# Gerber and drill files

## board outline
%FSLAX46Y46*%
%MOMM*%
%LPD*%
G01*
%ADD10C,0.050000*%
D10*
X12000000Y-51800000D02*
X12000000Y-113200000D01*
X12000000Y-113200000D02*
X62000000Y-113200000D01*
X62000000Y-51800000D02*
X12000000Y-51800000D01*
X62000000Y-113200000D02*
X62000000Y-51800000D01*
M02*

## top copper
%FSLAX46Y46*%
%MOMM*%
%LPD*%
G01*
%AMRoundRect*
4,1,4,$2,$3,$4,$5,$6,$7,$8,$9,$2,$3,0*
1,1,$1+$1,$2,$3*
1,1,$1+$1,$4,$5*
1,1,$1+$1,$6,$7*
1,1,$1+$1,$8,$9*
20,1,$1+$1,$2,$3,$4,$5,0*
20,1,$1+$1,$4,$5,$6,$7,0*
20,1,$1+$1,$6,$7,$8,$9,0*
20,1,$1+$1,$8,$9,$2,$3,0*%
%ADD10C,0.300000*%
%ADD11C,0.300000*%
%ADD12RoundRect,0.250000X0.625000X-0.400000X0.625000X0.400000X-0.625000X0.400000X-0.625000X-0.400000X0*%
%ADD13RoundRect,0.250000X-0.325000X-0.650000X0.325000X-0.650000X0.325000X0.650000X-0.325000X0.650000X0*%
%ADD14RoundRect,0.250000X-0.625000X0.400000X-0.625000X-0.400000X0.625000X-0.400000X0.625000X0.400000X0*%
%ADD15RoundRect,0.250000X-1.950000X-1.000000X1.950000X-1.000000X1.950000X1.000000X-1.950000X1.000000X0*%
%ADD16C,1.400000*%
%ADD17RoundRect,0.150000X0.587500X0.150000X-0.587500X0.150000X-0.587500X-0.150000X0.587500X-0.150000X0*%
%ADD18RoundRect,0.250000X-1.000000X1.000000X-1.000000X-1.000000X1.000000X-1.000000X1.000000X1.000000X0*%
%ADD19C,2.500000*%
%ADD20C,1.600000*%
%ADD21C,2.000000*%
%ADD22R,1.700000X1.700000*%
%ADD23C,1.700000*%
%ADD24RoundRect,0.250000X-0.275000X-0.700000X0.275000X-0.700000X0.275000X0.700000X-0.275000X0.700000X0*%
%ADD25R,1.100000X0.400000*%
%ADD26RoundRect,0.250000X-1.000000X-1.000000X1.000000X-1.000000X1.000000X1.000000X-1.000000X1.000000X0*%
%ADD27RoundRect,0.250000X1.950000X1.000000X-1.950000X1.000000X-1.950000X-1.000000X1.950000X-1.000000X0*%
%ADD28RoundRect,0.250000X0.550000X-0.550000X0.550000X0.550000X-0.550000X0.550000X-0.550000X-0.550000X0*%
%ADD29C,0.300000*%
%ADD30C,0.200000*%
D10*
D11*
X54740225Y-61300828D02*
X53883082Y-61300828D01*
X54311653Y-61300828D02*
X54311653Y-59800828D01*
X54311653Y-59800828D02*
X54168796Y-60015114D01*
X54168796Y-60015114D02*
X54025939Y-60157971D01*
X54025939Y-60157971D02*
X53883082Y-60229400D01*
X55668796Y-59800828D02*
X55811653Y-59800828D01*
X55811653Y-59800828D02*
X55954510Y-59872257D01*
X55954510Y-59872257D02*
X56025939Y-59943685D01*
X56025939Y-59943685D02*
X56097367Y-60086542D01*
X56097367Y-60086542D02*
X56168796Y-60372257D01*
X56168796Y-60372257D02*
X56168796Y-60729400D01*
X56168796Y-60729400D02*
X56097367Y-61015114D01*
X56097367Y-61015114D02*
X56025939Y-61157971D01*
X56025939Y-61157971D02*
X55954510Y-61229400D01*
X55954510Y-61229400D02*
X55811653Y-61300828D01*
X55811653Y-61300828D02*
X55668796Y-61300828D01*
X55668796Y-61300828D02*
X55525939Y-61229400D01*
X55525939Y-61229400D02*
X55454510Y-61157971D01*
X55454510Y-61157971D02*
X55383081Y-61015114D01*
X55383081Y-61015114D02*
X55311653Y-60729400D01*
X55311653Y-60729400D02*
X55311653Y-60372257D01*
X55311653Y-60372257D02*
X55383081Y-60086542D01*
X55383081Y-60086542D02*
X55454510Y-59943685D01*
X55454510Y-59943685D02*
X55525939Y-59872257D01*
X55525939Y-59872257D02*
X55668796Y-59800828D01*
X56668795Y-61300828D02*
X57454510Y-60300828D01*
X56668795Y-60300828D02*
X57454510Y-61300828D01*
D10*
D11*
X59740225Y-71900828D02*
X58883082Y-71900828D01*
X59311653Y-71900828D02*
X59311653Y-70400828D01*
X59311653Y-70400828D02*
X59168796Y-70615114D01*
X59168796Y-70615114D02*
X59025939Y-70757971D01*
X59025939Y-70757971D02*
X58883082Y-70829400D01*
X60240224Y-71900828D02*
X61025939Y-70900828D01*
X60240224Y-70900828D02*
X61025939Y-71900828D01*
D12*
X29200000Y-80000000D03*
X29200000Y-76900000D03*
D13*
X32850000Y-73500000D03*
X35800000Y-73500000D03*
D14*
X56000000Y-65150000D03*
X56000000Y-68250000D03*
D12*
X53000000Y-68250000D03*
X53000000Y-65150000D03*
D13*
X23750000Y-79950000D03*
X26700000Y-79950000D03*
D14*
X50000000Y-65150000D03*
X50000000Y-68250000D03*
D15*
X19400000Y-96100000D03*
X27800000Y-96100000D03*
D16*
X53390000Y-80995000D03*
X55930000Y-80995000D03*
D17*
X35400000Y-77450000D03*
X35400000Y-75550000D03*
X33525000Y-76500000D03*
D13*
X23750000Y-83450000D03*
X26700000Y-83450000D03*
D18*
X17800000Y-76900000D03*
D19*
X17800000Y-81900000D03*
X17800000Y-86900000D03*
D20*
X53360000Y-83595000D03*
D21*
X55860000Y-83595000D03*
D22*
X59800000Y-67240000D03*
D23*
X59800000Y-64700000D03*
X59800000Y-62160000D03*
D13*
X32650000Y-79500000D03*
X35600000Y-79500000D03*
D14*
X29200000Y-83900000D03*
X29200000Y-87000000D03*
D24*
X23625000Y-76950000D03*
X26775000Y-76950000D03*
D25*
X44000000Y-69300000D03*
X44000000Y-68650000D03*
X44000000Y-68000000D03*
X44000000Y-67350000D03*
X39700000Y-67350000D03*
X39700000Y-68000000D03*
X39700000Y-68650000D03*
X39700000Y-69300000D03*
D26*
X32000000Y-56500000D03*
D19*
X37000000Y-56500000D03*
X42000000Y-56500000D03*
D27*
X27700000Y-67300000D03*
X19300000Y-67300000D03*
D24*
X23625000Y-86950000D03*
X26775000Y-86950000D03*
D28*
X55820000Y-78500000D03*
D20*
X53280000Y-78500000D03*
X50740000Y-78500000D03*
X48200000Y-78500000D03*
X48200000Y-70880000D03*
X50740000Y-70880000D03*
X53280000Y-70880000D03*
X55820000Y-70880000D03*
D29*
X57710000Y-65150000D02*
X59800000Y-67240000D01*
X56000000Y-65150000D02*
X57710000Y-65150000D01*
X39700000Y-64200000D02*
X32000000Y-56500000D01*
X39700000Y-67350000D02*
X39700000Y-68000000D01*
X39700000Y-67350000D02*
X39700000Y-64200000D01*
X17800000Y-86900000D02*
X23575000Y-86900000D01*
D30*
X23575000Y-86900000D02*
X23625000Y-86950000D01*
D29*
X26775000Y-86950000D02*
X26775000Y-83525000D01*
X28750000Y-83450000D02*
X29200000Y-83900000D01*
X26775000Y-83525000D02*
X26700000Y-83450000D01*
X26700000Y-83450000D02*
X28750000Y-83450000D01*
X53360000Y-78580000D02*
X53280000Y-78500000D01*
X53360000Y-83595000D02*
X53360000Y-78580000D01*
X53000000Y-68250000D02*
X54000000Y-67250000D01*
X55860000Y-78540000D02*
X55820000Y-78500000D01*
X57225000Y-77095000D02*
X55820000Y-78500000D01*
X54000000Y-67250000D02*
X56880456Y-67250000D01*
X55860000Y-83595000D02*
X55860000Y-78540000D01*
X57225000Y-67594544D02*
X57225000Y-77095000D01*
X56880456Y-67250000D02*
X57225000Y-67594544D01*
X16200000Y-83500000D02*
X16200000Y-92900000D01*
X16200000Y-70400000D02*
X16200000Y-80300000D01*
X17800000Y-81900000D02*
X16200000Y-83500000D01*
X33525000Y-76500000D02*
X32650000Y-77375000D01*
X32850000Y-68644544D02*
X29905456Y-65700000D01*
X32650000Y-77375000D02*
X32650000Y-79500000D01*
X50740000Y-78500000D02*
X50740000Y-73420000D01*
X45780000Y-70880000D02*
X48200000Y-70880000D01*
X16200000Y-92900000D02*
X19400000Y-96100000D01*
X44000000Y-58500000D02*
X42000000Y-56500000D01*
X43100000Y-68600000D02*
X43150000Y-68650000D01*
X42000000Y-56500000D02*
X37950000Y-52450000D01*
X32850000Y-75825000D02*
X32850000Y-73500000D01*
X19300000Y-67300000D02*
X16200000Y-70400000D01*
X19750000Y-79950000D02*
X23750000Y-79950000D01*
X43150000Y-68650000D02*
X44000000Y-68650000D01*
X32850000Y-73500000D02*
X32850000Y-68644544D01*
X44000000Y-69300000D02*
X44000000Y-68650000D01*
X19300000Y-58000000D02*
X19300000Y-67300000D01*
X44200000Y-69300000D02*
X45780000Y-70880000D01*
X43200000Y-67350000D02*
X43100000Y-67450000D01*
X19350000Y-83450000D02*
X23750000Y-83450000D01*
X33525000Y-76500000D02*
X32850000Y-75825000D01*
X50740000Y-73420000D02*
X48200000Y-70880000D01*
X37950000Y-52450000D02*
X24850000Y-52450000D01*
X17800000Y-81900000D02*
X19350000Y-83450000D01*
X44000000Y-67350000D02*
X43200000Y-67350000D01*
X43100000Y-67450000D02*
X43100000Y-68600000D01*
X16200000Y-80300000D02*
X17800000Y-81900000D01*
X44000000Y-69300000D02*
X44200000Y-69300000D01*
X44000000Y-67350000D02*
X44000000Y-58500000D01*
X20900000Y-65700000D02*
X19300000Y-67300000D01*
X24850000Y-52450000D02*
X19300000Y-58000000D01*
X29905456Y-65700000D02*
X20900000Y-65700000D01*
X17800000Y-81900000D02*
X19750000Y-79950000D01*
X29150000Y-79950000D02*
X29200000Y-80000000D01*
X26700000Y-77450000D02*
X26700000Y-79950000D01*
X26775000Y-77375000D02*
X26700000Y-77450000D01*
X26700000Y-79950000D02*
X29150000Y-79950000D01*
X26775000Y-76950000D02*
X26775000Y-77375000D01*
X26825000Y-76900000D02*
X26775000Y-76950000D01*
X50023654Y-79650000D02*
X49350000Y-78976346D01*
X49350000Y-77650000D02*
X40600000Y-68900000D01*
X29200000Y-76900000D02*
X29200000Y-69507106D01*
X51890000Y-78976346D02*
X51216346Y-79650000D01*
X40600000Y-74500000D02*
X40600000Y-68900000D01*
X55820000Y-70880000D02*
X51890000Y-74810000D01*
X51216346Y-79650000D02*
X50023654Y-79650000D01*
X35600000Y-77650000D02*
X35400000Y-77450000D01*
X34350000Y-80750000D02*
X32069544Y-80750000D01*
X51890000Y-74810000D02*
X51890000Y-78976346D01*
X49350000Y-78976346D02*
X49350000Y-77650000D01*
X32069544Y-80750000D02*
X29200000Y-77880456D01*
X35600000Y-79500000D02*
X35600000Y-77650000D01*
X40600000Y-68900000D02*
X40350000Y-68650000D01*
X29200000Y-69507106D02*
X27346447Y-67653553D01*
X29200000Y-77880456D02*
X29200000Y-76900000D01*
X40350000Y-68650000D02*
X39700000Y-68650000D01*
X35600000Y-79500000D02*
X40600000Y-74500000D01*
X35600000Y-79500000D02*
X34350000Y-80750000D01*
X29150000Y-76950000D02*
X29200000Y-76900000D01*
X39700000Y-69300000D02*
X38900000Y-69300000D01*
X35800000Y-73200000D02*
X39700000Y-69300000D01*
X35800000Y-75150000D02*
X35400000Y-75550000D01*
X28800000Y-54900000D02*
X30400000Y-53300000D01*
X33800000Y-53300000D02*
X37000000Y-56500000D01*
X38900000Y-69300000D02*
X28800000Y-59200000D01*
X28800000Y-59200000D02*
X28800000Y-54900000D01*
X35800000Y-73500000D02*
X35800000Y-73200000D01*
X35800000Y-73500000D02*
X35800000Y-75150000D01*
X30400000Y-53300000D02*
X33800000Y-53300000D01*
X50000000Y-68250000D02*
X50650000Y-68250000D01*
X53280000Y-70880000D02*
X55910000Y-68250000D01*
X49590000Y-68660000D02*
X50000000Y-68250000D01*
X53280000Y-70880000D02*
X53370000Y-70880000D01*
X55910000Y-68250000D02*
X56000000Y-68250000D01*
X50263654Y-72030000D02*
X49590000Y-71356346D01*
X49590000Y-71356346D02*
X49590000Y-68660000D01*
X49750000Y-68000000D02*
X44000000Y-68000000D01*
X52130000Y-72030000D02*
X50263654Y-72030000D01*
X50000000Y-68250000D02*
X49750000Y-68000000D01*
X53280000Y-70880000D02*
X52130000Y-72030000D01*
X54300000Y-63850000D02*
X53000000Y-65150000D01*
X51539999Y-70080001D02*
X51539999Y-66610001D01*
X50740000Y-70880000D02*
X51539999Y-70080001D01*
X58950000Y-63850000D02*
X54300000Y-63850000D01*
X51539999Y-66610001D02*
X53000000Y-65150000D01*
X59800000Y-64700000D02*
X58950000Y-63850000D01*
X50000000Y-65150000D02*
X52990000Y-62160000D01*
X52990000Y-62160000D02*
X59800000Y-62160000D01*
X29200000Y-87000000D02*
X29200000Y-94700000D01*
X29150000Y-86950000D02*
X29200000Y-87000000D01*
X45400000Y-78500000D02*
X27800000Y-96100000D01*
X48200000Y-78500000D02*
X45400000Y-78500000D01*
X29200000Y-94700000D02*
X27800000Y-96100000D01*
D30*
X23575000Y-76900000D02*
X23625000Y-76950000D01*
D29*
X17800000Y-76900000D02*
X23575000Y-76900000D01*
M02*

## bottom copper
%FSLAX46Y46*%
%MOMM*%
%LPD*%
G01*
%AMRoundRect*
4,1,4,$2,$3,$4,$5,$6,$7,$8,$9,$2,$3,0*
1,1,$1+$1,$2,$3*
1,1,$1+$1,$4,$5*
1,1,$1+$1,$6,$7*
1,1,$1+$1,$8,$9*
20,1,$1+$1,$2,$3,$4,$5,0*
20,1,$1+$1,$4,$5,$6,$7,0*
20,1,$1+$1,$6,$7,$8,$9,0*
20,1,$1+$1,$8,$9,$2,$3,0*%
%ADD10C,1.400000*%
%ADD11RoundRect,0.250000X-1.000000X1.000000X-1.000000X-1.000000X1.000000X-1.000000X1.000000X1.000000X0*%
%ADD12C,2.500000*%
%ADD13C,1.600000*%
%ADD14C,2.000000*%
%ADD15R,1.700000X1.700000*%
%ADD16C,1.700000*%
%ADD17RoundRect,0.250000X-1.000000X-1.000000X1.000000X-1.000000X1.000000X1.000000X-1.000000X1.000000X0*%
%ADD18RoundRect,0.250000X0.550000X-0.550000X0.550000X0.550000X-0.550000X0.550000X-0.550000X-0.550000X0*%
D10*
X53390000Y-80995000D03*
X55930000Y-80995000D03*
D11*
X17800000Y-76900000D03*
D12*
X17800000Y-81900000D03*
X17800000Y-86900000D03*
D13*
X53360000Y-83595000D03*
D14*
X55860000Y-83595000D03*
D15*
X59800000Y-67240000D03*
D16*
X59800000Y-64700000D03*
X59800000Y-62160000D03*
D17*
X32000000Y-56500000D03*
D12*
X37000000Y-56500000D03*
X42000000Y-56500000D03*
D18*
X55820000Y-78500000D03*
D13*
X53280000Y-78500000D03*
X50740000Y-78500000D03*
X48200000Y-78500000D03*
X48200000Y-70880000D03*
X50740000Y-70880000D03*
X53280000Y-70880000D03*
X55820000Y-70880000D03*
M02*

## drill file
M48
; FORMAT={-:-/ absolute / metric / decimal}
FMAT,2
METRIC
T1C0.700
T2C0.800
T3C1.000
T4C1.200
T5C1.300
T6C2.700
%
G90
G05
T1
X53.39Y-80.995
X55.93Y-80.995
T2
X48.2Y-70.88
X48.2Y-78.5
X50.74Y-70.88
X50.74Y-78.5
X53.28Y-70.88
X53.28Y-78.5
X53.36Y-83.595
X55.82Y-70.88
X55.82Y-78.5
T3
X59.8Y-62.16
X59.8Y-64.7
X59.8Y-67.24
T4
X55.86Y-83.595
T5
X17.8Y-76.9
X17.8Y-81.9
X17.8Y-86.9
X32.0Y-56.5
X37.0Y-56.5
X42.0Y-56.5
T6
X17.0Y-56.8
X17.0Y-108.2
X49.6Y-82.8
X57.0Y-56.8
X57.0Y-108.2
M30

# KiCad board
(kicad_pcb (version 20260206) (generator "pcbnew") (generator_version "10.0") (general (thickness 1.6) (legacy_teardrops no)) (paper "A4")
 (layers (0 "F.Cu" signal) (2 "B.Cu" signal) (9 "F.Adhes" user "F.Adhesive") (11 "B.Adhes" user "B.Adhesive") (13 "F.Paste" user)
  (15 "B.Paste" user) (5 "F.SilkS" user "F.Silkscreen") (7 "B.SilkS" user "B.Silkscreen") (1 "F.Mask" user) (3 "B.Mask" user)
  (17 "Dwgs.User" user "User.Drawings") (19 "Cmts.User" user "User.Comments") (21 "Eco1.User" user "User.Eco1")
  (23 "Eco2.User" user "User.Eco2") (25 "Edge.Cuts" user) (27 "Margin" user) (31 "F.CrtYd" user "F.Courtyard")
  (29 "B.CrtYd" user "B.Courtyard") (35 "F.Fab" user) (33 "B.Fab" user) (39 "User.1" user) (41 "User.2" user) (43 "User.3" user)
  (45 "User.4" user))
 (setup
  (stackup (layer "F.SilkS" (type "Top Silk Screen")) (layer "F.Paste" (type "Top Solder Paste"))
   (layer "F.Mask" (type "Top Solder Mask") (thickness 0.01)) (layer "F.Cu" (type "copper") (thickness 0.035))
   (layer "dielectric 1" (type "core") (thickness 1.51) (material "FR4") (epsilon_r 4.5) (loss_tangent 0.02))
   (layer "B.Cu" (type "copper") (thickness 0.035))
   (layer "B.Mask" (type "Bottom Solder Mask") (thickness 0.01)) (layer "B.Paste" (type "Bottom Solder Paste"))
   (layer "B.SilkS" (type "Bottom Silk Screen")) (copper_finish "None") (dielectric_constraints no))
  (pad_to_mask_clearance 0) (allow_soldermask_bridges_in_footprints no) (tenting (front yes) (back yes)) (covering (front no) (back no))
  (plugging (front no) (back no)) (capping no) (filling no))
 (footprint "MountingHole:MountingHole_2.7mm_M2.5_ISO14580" (layer "F.Cu") (at 57 56.8 -90)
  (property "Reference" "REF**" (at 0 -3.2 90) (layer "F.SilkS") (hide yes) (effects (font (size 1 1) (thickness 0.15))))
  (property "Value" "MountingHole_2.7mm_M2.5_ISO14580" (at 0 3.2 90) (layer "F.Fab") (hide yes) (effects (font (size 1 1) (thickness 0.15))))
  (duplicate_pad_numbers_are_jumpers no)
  (pad "" np_thru_hole circle (at 0 0 270) (size 2.7 2.7) (drill 2.7) (layers "*.Cu" "*.Mask")))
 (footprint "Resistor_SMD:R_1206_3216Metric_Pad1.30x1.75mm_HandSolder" (layer "F.Cu") (at 29.2 78.45 90)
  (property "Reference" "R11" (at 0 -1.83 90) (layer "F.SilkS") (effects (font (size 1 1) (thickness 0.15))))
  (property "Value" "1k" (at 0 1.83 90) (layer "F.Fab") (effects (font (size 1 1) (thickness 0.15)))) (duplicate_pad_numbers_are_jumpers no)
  (pad "1" smd roundrect (at -1.55 0 90) (size 1.3 1.75) (layers "F.Cu" "F.Mask" "F.Paste") (roundrect_rratio 0.192308)
   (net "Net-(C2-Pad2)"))
  (pad "2" smd roundrect (at 1.55 0 90) (size 1.3 1.75) (layers "F.Cu" "F.Mask" "F.Paste") (roundrect_rratio 0.192308) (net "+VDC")))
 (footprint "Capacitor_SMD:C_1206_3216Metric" (layer "F.Cu") (at 34.325 73.5)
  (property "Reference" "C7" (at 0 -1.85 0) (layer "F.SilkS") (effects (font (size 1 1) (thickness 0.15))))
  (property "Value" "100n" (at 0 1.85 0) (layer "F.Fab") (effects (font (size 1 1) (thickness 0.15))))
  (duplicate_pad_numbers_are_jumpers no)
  (pad "1" smd roundrect (at -1.475 0) (size 1.15 1.8) (layers "F.Cu" "F.Mask" "F.Paste") (roundrect_rratio 0.217391) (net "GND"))
  (pad "2" smd roundrect (at 1.475 0) (size 1.15 1.8) (layers "F.Cu" "F.Mask" "F.Paste") (roundrect_rratio 0.217391) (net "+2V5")))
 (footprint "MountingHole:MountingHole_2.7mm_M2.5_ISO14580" (layer "F.Cu") (at 49.6 82.8 180)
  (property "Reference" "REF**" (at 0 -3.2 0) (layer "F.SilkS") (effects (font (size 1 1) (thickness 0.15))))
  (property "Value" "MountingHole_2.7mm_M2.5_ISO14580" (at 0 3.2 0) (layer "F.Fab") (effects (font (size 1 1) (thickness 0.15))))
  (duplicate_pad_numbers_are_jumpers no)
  (pad "" np_thru_hole circle (at 0 0 180) (size 2.7 2.7) (drill 2.7) (layers "*.Cu" "*.Mask")))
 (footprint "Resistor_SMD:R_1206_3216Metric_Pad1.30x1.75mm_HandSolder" (layer "F.Cu") (at 56 66.7 -90)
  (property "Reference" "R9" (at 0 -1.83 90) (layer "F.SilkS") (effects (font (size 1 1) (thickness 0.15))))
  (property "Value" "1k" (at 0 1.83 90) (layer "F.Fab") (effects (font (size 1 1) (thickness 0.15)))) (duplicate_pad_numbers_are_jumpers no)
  (pad "1" smd roundrect (at -1.55 0 270) (size 1.3 1.75) (layers "F.Cu" "F.Mask" "F.Paste") (roundrect_rratio 0.192308)
   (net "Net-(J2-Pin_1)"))
  (pad "2" smd roundrect (at 1.55 0 270) (size 1.3 1.75) (layers "F.Cu" "F.Mask" "F.Paste") (roundrect_rratio 0.192308)
   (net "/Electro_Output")))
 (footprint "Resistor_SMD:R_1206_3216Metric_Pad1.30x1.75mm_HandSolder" (layer "F.Cu") (at 53 66.7 90)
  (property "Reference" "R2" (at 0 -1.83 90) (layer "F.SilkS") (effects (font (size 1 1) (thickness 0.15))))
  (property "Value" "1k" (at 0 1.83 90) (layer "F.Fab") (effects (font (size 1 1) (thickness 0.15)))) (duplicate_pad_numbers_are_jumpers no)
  (pad "1" smd roundrect (at -1.55 0 90) (size 1.3 1.75) (layers "F.Cu" "F.Mask" "F.Paste") (roundrect_rratio 0.192308)
   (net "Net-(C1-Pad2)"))
  (pad "2" smd roundrect (at 1.55 0 90) (size 1.3 1.75) (layers "F.Cu" "F.Mask" "F.Paste") (roundrect_rratio 0.192308)
   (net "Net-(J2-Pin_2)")))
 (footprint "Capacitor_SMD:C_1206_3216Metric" (layer "F.Cu") (at 25.225 79.95)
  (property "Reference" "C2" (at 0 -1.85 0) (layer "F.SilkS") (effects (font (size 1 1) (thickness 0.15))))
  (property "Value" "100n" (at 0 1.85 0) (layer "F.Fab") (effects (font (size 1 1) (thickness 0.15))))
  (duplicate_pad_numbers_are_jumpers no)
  (pad "1" smd roundrect (at -1.475 0) (size 1.15 1.8) (layers "F.Cu" "F.Mask" "F.Paste") (roundrect_rratio 0.217391) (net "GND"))
  (pad "2" smd roundrect (at 1.475 0) (size 1.15 1.8) (layers "F.Cu" "F.Mask" "F.Paste") (roundrect_rratio 0.217391) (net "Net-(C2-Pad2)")))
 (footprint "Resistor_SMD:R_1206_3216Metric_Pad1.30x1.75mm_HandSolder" (layer "F.Cu") (at 50 66.7 -90)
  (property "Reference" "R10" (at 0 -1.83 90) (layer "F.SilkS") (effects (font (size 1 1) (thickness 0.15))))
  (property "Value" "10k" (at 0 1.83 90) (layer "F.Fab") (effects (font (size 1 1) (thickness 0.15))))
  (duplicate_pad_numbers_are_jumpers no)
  (pad "1" smd roundrect (at -1.55 0 270) (size 1.3 1.75) (layers "F.Cu" "F.Mask" "F.Paste") (roundrect_rratio 0.192308)
   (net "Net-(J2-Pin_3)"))
  (pad "2" smd roundrect (at 1.55 0 270) (size 1.3 1.75) (layers "F.Cu" "F.Mask" "F.Paste") (roundrect_rratio 0.192308)
   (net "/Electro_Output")))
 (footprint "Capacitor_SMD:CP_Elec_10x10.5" (layer "F.Cu") (at 23.6 96.1)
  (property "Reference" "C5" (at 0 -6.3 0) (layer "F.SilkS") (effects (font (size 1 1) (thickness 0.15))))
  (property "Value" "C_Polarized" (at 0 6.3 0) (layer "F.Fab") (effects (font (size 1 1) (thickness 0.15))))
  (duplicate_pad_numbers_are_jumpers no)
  (pad "1" smd roundrect (at -4.2 0) (size 4.4 2.5) (layers "F.Cu" "F.Mask" "F.Paste") (roundrect_rratio 0.1) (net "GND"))
  (pad "2" smd roundrect (at 4.2 0) (size 4.4 2.5) (layers "F.Cu" "F.Mask" "F.Paste") (roundrect_rratio 0.1) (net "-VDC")))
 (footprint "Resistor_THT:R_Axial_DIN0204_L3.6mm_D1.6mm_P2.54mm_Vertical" (layer "F.Cu") (at 53.39 80.995)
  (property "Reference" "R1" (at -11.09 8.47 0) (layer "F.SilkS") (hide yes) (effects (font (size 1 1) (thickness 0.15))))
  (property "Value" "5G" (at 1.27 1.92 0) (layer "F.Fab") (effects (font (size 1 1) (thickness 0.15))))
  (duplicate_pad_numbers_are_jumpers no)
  (pad "1" thru_hole circle (at 0 0) (size 1.4 1.4) (drill 0.7) (layers "*.Cu" "*.Mask") (remove_unused_layers no) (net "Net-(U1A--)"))
  (pad "2" thru_hole circle (at 2.54 0) (size 1.4 1.4) (drill 0.7) (layers "*.Cu" "*.Mask") (remove_unused_layers no) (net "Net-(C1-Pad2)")))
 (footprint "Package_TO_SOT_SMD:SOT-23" (layer "F.Cu") (at 34.4625 76.5 180)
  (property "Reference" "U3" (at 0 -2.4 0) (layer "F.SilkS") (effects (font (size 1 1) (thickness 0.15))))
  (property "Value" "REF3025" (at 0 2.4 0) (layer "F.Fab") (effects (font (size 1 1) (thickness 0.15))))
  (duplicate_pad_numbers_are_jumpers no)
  (pad "1" smd roundrect (at -0.9375 -0.95 180) (size 1.475 0.6) (layers "F.Cu" "F.Mask" "F.Paste") (roundrect_rratio 0.25) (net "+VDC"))
  (pad "2" smd roundrect (at -0.9375 0.95 180) (size 1.475 0.6) (layers "F.Cu" "F.Mask" "F.Paste") (roundrect_rratio 0.25) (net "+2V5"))
  (pad "3" smd roundrect (at 0.9375 0 180) (size 1.475 0.6) (layers "F.Cu" "F.Mask" "F.Paste") (roundrect_rratio 0.25) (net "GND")))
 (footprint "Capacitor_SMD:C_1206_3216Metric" (layer "F.Cu") (at 25.225 83.45)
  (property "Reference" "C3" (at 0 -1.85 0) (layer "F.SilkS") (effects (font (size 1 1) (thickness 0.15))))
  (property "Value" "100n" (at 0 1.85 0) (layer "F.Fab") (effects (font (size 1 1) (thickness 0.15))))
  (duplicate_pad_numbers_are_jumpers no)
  (pad "1" smd roundrect (at -1.475 0) (size 1.15 1.8) (layers "F.Cu" "F.Mask" "F.Paste") (roundrect_rratio 0.217391) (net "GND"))
  (pad "2" smd roundrect (at 1.475 0) (size 1.15 1.8) (layers "F.Cu" "F.Mask" "F.Paste") (roundrect_rratio 0.217391) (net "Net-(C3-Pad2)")))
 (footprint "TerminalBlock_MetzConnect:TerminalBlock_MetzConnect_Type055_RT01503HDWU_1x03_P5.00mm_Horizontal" (layer "F.Cu")
  (at 17.8 76.9 -90)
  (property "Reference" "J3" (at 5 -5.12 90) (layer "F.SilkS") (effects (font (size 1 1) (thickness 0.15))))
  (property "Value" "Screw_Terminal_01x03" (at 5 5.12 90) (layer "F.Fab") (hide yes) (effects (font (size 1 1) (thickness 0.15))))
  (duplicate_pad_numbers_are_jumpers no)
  (pad "1" thru_hole roundrect (at 0 0 270) (size 2.5 2.5) (drill 1.3) (layers "*.Cu" "*.Mask") (remove_unused_layers no)
   (roundrect_rratio 0.1) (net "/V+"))
  (pad "2" thru_hole circle (at 5 0 270) (size 2.5 2.5) (drill 1.3) (layers "*.Cu" "*.Mask") (remove_unused_layers no) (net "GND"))
  (pad "3" thru_hole circle (at 10 0 270) (size 2.5 2.5) (drill 1.3) (layers "*.Cu" "*.Mask") (remove_unused_layers no) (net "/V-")))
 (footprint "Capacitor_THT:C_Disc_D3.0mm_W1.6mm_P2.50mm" (layer "F.Cu") (at 53.36 83.595)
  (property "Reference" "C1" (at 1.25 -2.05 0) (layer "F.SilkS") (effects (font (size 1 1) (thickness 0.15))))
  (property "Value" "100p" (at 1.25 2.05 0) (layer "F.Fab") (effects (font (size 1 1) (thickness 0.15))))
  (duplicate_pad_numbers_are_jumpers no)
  (pad "1" thru_hole circle (at 0 0) (size 1.6 1.6) (drill 0.8) (layers "*.Cu" "*.Mask") (remove_unused_layers no) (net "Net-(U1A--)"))
  (pad "2" thru_hole circle (at 2.5 0) (size 2 2) (drill 1.2) (layers "*.Cu" "*.Mask") (remove_unused_layers no) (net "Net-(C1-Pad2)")))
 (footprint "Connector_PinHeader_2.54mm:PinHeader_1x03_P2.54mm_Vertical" (layer "F.Cu") (at 59.8 67.24 180)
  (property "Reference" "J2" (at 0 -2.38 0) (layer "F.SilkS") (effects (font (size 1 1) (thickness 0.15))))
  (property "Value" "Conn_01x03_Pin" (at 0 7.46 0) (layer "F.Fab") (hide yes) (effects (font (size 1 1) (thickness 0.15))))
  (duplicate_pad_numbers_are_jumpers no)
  (pad "1" thru_hole rect (at 0 0 180) (size 1.7 1.7) (drill 1) (layers "*.Cu" "*.Mask") (remove_unused_layers no) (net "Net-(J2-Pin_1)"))
  (pad "2" thru_hole circle (at 0 2.54 180) (size 1.7 1.7) (drill 1) (layers "*.Cu" "*.Mask") (remove_unused_layers no)
   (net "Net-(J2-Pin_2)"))
  (pad "3" thru_hole circle (at 0 5.08 180) (size 1.7 1.7) (drill 1) (layers "*.Cu" "*.Mask") (remove_unused_layers no)
   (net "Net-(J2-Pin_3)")))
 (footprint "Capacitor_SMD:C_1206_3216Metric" (layer "F.Cu") (at 34.125 79.5)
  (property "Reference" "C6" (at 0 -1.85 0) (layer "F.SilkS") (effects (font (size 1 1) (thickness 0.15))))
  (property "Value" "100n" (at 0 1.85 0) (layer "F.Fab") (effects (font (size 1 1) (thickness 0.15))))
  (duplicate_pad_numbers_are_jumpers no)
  (pad "1" smd roundrect (at -1.475 0) (size 1.15 1.8) (layers "F.Cu" "F.Mask" "F.Paste") (roundrect_rratio 0.217391) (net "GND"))
  (pad "2" smd roundrect (at 1.475 0) (size 1.15 1.8) (layers "F.Cu" "F.Mask" "F.Paste") (roundrect_rratio 0.217391) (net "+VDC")))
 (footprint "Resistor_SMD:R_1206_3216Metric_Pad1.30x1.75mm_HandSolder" (layer "F.Cu") (at 29.2 85.45 -90)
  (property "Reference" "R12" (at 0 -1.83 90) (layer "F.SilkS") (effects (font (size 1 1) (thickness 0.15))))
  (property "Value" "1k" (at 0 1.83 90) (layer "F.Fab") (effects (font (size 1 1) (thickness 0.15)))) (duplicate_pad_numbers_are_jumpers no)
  (pad "1" smd roundrect (at -1.55 0 270) (size 1.3 1.75) (layers "F.Cu" "F.Mask" "F.Paste") (roundrect_rratio 0.192308)
   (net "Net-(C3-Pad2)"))
  (pad "2" smd roundrect (at 1.55 0 270) (size 1.3 1.75) (layers "F.Cu" "F.Mask" "F.Paste") (roundrect_rratio 0.192308) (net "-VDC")))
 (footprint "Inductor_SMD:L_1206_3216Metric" (layer "F.Cu") (at 25.2 76.95)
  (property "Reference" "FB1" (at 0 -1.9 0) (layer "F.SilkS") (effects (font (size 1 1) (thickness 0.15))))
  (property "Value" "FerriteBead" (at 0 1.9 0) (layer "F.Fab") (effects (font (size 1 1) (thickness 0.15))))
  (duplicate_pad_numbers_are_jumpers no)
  (pad "1" smd roundrect (at -1.575 0) (size 1.05 1.9) (layers "F.Cu" "F.Mask" "F.Paste") (roundrect_rratio 0.238095) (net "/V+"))
  (pad "2" smd roundrect (at 1.575 0) (size 1.05 1.9) (layers "F.Cu" "F.Mask" "F.Paste") (roundrect_rratio 0.238095) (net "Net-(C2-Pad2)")))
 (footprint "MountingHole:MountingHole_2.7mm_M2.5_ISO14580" (layer "F.Cu") (at 57 108.2 -90)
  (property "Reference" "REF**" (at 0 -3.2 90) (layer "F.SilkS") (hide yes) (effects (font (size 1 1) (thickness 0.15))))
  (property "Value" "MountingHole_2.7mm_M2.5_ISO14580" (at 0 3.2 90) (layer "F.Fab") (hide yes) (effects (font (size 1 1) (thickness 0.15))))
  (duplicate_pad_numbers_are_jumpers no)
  (pad "" np_thru_hole circle (at 0 0 270) (size 2.7 2.7) (drill 2.7) (layers "*.Cu" "*.Mask")))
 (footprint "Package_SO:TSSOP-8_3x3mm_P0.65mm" (layer "F.Cu") (at 41.85 68.325 180)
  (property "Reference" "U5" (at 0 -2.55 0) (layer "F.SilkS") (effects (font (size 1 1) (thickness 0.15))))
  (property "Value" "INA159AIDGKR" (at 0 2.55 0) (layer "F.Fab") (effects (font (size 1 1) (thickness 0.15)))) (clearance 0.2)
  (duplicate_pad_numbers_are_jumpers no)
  (pad "1" smd rect (at -2.15 -0.975 180) (size 1.1 0.4) (layers "F.Cu" "F.Mask" "F.Paste") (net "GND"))
  (pad "2" smd rect (at -2.15 -0.325 180) (size 1.1 0.4) (layers "F.Cu" "F.Mask" "F.Paste") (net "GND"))
  (pad "3" smd rect (at -2.15 0.325 180) (size 1.1 0.4) (layers "F.Cu" "F.Mask" "F.Paste") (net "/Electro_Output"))
  (pad "4" smd rect (at -2.15 0.975 180) (size 1.1 0.4) (layers "F.Cu" "F.Mask" "F.Paste") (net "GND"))
  (pad "5" smd rect (at 2.15 0.975 180) (size 1.1 0.4) (layers "F.Cu" "F.Mask" "F.Paste") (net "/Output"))
  (pad "6" smd rect (at 2.15 0.325 180) (size 1.1 0.4) (layers "F.Cu" "F.Mask" "F.Paste") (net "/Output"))
  (pad "7" smd rect (at 2.15 -0.325 180) (size 1.1 0.4) (layers "F.Cu" "F.Mask" "F.Paste") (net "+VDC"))
  (pad "8" smd rect (at 2.15 -0.975 180) (size 1.1 0.4) (layers "F.Cu" "F.Mask" "F.Paste") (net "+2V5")))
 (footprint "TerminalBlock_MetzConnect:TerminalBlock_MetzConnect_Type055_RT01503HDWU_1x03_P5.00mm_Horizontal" (layer "F.Cu") (at 32 56.5)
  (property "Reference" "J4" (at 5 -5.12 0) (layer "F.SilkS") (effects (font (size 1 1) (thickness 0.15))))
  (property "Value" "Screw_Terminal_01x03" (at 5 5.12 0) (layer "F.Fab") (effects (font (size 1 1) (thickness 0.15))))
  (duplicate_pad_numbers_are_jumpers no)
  (pad "1" thru_hole roundrect (at 0 0) (size 2.5 2.5) (drill 1.3) (layers "*.Cu" "*.Mask") (remove_unused_layers no) (roundrect_rratio 0.1)
   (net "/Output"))
  (pad "2" thru_hole circle (at 5 0) (size 2.5 2.5) (drill 1.3) (layers "*.Cu" "*.Mask") (remove_unused_layers no) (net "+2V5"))
  (pad "3" thru_hole circle (at 10 0) (size 2.5 2.5) (drill 1.3) (layers "*.Cu" "*.Mask") (remove_unused_layers no) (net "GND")))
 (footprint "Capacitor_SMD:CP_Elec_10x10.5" (layer "F.Cu") (at 23.5 67.3 180)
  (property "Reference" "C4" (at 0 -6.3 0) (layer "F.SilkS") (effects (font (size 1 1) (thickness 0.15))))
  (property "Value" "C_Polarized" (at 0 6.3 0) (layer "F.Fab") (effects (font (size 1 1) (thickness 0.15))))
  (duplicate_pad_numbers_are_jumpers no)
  (pad "1" smd roundrect (at -4.2 0 180) (size 4.4 2.5) (layers "F.Cu" "F.Mask" "F.Paste") (roundrect_rratio 0.1) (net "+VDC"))
  (pad "2" smd roundrect (at 4.2 0 180) (size 4.4 2.5) (layers "F.Cu" "F.Mask" "F.Paste") (roundrect_rratio 0.1) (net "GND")))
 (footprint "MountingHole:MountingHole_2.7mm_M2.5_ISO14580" (layer "F.Cu") (at 17 108.2 -90)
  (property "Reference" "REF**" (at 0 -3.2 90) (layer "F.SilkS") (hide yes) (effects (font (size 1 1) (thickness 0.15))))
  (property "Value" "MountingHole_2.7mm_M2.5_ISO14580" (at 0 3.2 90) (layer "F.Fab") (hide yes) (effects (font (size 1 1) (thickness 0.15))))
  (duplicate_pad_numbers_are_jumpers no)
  (pad "" np_thru_hole circle (at 0 0 270) (size 2.7 2.7) (drill 2.7) (layers "*.Cu" "*.Mask")))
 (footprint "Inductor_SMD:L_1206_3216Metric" (layer "F.Cu") (at 25.2 86.95)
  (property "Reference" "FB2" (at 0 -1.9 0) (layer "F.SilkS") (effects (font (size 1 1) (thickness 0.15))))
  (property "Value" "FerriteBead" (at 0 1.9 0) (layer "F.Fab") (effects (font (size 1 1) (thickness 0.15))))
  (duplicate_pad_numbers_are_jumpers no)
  (pad "1" smd roundrect (at -1.575 0) (size 1.05 1.9) (layers "F.Cu" "F.Mask" "F.Paste") (roundrect_rratio 0.238095) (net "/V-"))
  (pad "2" smd roundrect (at 1.575 0) (size 1.05 1.9) (layers "F.Cu" "F.Mask" "F.Paste") (roundrect_rratio 0.238095) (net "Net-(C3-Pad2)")))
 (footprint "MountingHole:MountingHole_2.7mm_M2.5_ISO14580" (layer "F.Cu") (at 17 56.8 -90)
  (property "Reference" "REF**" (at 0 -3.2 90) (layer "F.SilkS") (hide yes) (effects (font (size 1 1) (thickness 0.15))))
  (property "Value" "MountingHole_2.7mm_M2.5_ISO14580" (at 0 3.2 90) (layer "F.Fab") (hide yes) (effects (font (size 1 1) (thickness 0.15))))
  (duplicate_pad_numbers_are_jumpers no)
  (pad "" np_thru_hole circle (at 0 0 270) (size 2.7 2.7) (drill 2.7) (layers "*.Cu" "*.Mask")))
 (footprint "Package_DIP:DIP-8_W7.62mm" (layer "B.Cu") (at 55.82 78.5 90)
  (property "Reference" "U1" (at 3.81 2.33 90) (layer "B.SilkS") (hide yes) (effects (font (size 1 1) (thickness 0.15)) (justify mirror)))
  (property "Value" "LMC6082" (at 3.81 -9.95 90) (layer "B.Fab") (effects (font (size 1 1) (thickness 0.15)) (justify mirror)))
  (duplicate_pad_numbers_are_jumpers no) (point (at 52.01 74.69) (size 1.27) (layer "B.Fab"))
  (pad "1" thru_hole roundrect (at 0 0 90) (size 1.6 1.6) (drill 0.8) (layers "*.Cu" "*.Mask") (remove_unused_layers no)
   (roundrect_rratio 0.15625) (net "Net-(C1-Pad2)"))
  (pad "2" thru_hole circle (at 0 -2.54 90) (size 1.6 1.6) (drill 0.8) (layers "*.Cu" "*.Mask") (remove_unused_layers no)
   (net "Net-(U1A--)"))
  (pad "3" thru_hole circle (at 0 -5.08 90) (size 1.6 1.6) (drill 0.8) (layers "*.Cu" "*.Mask") (remove_unused_layers no) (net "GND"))
  (pad "4" thru_hole circle (at 0 -7.62 90) (size 1.6 1.6) (drill 0.8) (layers "*.Cu" "*.Mask") (remove_unused_layers no) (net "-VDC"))
  (pad "5" thru_hole circle (at 7.62 -7.62 90) (size 1.6 1.6) (drill 0.8) (layers "*.Cu" "*.Mask") (remove_unused_layers no) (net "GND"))
  (pad "6" thru_hole circle (at 7.62 -5.08 90) (size 1.6 1.6) (drill 0.8) (layers "*.Cu" "*.Mask") (remove_unused_layers no)
   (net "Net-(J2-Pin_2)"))
  (pad "7" thru_hole circle (at 7.62 -2.54 90) (size 1.6 1.6) (drill 0.8) (layers "*.Cu" "*.Mask") (remove_unused_layers no)
   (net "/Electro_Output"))
  (pad "8" thru_hole circle (at 7.62 0 90) (size 1.6 1.6) (drill 0.8) (layers "*.Cu" "*.Mask") (remove_unused_layers no) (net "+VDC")))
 (gr_line (start 12 51.8) (end 12 113.2) (stroke (width 0.05) (type default)) (layer "Edge.Cuts"))
 (gr_line (start 12 113.2) (end 62 113.2) (stroke (width 0.05) (type default)) (layer "Edge.Cuts"))
 (gr_line (start 62 51.8) (end 12 51.8) (stroke (width 0.05) (type default)) (layer "Edge.Cuts"))
 (gr_line (start 62 113.2) (end 62 51.8) (stroke (width 0.05) (type default)) (layer "Edge.Cuts"))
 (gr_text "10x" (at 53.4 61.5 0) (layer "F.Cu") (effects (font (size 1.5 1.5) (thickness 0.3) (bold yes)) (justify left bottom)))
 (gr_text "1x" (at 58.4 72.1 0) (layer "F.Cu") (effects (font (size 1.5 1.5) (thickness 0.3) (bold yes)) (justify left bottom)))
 (segment (start 57.71 65.15) (end 59.8 67.24) (width 0.3) (layer "F.Cu") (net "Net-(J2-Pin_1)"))
 (segment (start 56 65.15) (end 57.71 65.15) (width 0.3) (layer "F.Cu") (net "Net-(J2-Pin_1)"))
 (segment (start 39.7 64.2) (end 32 56.5) (width 0.3) (layer "F.Cu") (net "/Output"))
 (segment (start 39.7 67.35) (end 39.7 68) (width 0.3) (layer "F.Cu") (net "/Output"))
 (segment (start 39.7 67.35) (end 39.7 64.2) (width 0.3) (layer "F.Cu") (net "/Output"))
 (segment (start 17.8 86.9) (end 23.575 86.9) (width 0.3) (layer "F.Cu") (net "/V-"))
 (segment (start 23.575 86.9) (end 23.625 86.95) (width 0.2) (layer "F.Cu") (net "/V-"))
 (segment (start 26.775 86.95) (end 26.775 83.525) (width 0.3) (layer "F.Cu") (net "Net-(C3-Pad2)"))
 (segment (start 28.75 83.45) (end 29.2 83.9) (width 0.3) (layer "F.Cu") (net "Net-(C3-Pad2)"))
 (segment (start 26.775 83.525) (end 26.7 83.45) (width 0.3) (layer "F.Cu") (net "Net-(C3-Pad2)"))
 (segment (start 26.7 83.45) (end 28.75 83.45) (width 0.3) (layer "F.Cu") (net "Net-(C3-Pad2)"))
 (segment (start 53.36 78.58) (end 53.28 78.5) (width 0.3) (layer "F.Cu") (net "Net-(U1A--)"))
 (segment (start 53.36 83.595) (end 53.36 78.58) (width 0.3) (layer "F.Cu") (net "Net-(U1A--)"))
 (segment (start 53 68.25) (end 54 67.25) (width 0.3) (layer "F.Cu") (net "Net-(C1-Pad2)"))
 (segment (start 55.86 78.54) (end 55.82 78.5) (width 0.3) (layer "F.Cu") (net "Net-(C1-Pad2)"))
 (segment (start 57.225 77.095) (end 55.82 78.5) (width 0.3) (layer "F.Cu") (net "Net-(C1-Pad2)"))
 (segment (start 54 67.25) (end 56.880456 67.25) (width 0.3) (layer "F.Cu") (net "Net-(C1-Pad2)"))
 (segment (start 55.86 83.595) (end 55.86 78.54) (width 0.3) (layer "F.Cu") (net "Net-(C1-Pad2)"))
 (segment (start 57.225 67.594544) (end 57.225 77.095) (width 0.3) (layer "F.Cu") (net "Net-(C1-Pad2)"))
 (segment (start 56.880456 67.25) (end 57.225 67.594544) (width 0.3) (layer "F.Cu") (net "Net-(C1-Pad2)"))
 (segment (start 16.2 83.5) (end 16.2 92.9) (width 0.3) (layer "F.Cu") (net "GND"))
 (segment (start 16.2 70.4) (end 16.2 80.3) (width 0.3) (layer "F.Cu") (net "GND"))
 (segment (start 17.8 81.9) (end 16.2 83.5) (width 0.3) (layer "F.Cu") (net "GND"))
 (segment (start 33.525 76.5) (end 32.65 77.375) (width 0.3) (layer "F.Cu") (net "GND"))
 (segment (start 32.85 68.644544) (end 29.905456 65.7) (width 0.3) (layer "F.Cu") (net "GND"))
 (segment (start 32.65 77.375) (end 32.65 79.5) (width 0.3) (layer "F.Cu") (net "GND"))
 (segment (start 50.74 78.5) (end 50.74 73.42) (width 0.3) (layer "F.Cu") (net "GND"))
 (segment (start 45.78 70.88) (end 48.2 70.88) (width 0.3) (layer "F.Cu") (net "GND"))
 (segment (start 16.2 92.9) (end 19.4 96.1) (width 0.3) (layer "F.Cu") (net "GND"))
 (segment (start 44 58.5) (end 42 56.5) (width 0.3) (layer "F.Cu") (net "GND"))
 (segment (start 43.1 68.6) (end 43.15 68.65) (width 0.3) (layer "F.Cu") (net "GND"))
 (segment (start 42 56.5) (end 37.95 52.45) (width 0.3) (layer "F.Cu") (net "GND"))
 (segment (start 32.85 75.825) (end 32.85 73.5) (width 0.3) (layer "F.Cu") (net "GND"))
 (segment (start 19.3 67.3) (end 16.2 70.4) (width 0.3) (layer "F.Cu") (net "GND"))
 (segment (start 19.75 79.95) (end 23.75 79.95) (width 0.3) (layer "F.Cu") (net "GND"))
 (segment (start 43.15 68.65) (end 44 68.65) (width 0.3) (layer "F.Cu") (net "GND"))
 (segment (start 32.85 73.5) (end 32.85 68.644544) (width 0.3) (layer "F.Cu") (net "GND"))
 (segment (start 44 69.3) (end 44 68.65) (width 0.3) (layer "F.Cu") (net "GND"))
 (segment (start 19.3 58) (end 19.3 67.3) (width 0.3) (layer "F.Cu") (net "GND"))
 (segment (start 44.2 69.3) (end 45.78 70.88) (width 0.3) (layer "F.Cu") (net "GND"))
 (segment (start 43.2 67.35) (end 43.1 67.45) (width 0.3) (layer "F.Cu") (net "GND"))
 (segment (start 19.35 83.45) (end 23.75 83.45) (width 0.3) (layer "F.Cu") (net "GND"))
 (segment (start 33.525 76.5) (end 32.85 75.825) (width 0.3) (layer "F.Cu") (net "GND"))
 (segment (start 50.74 73.42) (end 48.2 70.88) (width 0.3) (layer "F.Cu") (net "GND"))
 (segment (start 37.95 52.45) (end 24.85 52.45) (width 0.3) (layer "F.Cu") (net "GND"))
 (segment (start 17.8 81.9) (end 19.35 83.45) (width 0.3) (layer "F.Cu") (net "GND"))
 (segment (start 44 67.35) (end 43.2 67.35) (width 0.3) (layer "F.Cu") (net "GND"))
 (segment (start 43.1 67.45) (end 43.1 68.6) (width 0.3) (layer "F.Cu") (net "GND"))
 (segment (start 16.2 80.3) (end 17.8 81.9) (width 0.3) (layer "F.Cu") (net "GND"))
 (segment (start 44 69.3) (end 44.2 69.3) (width 0.3) (layer "F.Cu") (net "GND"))
 (segment (start 44 67.35) (end 44 58.5) (width 0.3) (layer "F.Cu") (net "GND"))
 (segment (start 20.9 65.7) (end 19.3 67.3) (width 0.3) (layer "F.Cu") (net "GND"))
 (segment (start 24.85 52.45) (end 19.3 58) (width 0.3) (layer "F.Cu") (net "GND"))
 (segment (start 29.905456 65.7) (end 20.9 65.7) (width 0.3) (layer "F.Cu") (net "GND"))
 (segment (start 17.8 81.9) (end 19.75 79.95) (width 0.3) (layer "F.Cu") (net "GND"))
 (segment (start 29.15 79.95) (end 29.2 80) (width 0.3) (layer "F.Cu") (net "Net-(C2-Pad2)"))
 (segment (start 26.7 77.45) (end 26.7 79.95) (width 0.3) (layer "F.Cu") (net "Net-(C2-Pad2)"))
 (segment (start 26.775 77.375) (end 26.7 77.45) (width 0.3) (layer "F.Cu") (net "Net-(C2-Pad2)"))
 (segment (start 26.7 79.95) (end 29.15 79.95) (width 0.3) (layer "F.Cu") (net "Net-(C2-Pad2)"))
 (segment (start 26.775 76.95) (end 26.775 77.375) (width 0.3) (layer "F.Cu") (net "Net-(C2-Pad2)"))
 (segment (start 26.825 76.9) (end 26.775 76.95) (width 0.3) (layer "F.Cu") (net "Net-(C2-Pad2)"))
 (segment (start 50.023654 79.65) (end 49.35 78.976346) (width 0.3) (layer "F.Cu") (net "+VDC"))
 (segment (start 49.35 77.65) (end 40.6 68.9) (width 0.3) (layer "F.Cu") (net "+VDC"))
 (segment (start 29.2 76.9) (end 29.2 69.507106) (width 0.3) (layer "F.Cu") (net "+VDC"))
 (segment (start 51.89 78.976346) (end 51.216346 79.65) (width 0.3) (layer "F.Cu") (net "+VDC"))
 (segment (start 40.6 74.5) (end 40.6 68.9) (width 0.3) (layer "F.Cu") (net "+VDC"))
 (segment (start 55.82 70.88) (end 51.89 74.81) (width 0.3) (layer "F.Cu") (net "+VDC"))
 (segment (start 51.216346 79.65) (end 50.023654 79.65) (width 0.3) (layer "F.Cu") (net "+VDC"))
 (segment (start 35.6 77.65) (end 35.4 77.45) (width 0.3) (layer "F.Cu") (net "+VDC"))
 (segment (start 34.35 80.75) (end 32.069544 80.75) (width 0.3) (layer "F.Cu") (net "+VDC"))
 (segment (start 51.89 74.81) (end 51.89 78.976346) (width 0.3) (layer "F.Cu") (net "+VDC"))
 (segment (start 49.35 78.976346) (end 49.35 77.65) (width 0.3) (layer "F.Cu") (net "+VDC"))
 (segment (start 32.069544 80.75) (end 29.2 77.880456) (width 0.3) (layer "F.Cu") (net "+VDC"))
 (segment (start 35.6 79.5) (end 35.6 77.65) (width 0.3) (layer "F.Cu") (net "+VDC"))
 (segment (start 40.6 68.9) (end 40.35 68.65) (width 0.3) (layer "F.Cu") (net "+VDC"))
 (segment (start 29.2 69.507106) (end 27.346447 67.653553) (width 0.3) (layer "F.Cu") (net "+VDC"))
 (segment (start 29.2 77.880456) (end 29.2 76.9) (width 0.3) (layer "F.Cu") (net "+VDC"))
 (segment (start 40.35 68.65) (end 39.7 68.65) (width 0.3) (layer "F.Cu") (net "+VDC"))
 (segment (start 35.6 79.5) (end 40.6 74.5) (width 0.3) (layer "F.Cu") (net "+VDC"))
 (segment (start 35.6 79.5) (end 34.35 80.75) (width 0.3) (layer "F.Cu") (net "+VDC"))
 (segment (start 29.15 76.95) (end 29.2 76.9) (width 0.3) (layer "F.Cu") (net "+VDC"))
 (segment (start 39.7 69.3) (end 38.9 69.3) (width 0.3) (layer "F.Cu") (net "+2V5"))
 (segment (start 35.8 73.2) (end 39.7 69.3) (width 0.3) (layer "F.Cu") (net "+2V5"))
 (segment (start 35.8 75.15) (end 35.4 75.55) (width 0.3) (layer "F.Cu") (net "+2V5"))
 (segment (start 28.8 54.9) (end 30.4 53.3) (width 0.3) (layer "F.Cu") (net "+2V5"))
 (segment (start 33.8 53.3) (end 37 56.5) (width 0.3) (layer "F.Cu") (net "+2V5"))
 (segment (start 38.9 69.3) (end 28.8 59.2) (width 0.3) (layer "F.Cu") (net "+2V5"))
 (segment (start 28.8 59.2) (end 28.8 54.9) (width 0.3) (layer "F.Cu") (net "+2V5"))
 (segment (start 35.8 73.5) (end 35.8 73.2) (width 0.3) (layer "F.Cu") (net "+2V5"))
 (segment (start 35.8 73.5) (end 35.8 75.15) (width 0.3) (layer "F.Cu") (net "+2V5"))
 (segment (start 30.4 53.3) (end 33.8 53.3) (width 0.3) (layer "F.Cu") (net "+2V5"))
 (segment (start 50 68.25) (end 50.65 68.25) (width 0.3) (layer "F.Cu") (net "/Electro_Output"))
 (segment (start 53.28 70.88) (end 55.91 68.25) (width 0.3) (layer "F.Cu") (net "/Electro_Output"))
 (segment (start 49.59 68.66) (end 50 68.25) (width 0.3) (layer "F.Cu") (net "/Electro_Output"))
 (segment (start 53.28 70.88) (end 53.37 70.88) (width 0.3) (layer "F.Cu") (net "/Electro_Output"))
 (segment (start 55.91 68.25) (end 56 68.25) (width 0.3) (layer "F.Cu") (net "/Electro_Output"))
 (segment (start 50.263654 72.03) (end 49.59 71.356346) (width 0.3) (layer "F.Cu") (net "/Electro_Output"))
 (segment (start 49.59 71.356346) (end 49.59 68.66) (width 0.3) (layer "F.Cu") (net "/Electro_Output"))
 (segment (start 49.75 68) (end 44 68) (width 0.3) (layer "F.Cu") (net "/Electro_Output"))
 (segment (start 52.13 72.03) (end 50.263654 72.03) (width 0.3) (layer "F.Cu") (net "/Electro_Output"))
 (segment (start 50 68.25) (end 49.75 68) (width 0.3) (layer "F.Cu") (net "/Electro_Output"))
 (segment (start 53.28 70.88) (end 52.13 72.03) (width 0.3) (layer "F.Cu") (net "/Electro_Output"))
 (segment (start 54.3 63.85) (end 53 65.15) (width 0.3) (layer "F.Cu") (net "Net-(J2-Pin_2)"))
 (segment (start 51.539999 70.080001) (end 51.539999 66.610001) (width 0.3) (layer "F.Cu") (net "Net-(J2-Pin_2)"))
 (segment (start 50.74 70.88) (end 51.539999 70.080001) (width 0.3) (layer "F.Cu") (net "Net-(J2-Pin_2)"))
 (segment (start 58.95 63.85) (end 54.3 63.85) (width 0.3) (layer "F.Cu") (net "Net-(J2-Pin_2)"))
 (segment (start 51.539999 66.610001) (end 53 65.15) (width 0.3) (layer "F.Cu") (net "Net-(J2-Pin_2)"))
 (segment (start 59.8 64.7) (end 58.95 63.85) (width 0.3) (layer "F.Cu") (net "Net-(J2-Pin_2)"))
 (segment (start 50 65.15) (end 52.99 62.16) (width 0.3) (layer "F.Cu") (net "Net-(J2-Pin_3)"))
 (segment (start 52.99 62.16) (end 59.8 62.16) (width 0.3) (layer "F.Cu") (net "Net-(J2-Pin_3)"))
 (segment (start 29.2 87) (end 29.2 94.7) (width 0.3) (layer "F.Cu") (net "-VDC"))
 (segment (start 29.15 86.95) (end 29.2 87) (width 0.3) (layer "F.Cu") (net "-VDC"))
 (segment (start 45.4 78.5) (end 27.8 96.1) (width 0.3) (layer "F.Cu") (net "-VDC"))
 (segment (start 48.2 78.5) (end 45.4 78.5) (width 0.3) (layer "F.Cu") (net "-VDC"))
 (segment (start 29.2 94.7) (end 27.8 96.1) (width 0.3) (layer "F.Cu") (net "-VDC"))
 (segment (start 23.575 76.9) (end 23.625 76.95) (width 0.2) (layer "F.Cu") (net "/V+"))
 (segment (start 17.8 76.9) (end 23.575 76.9) (width 0.3) (layer "F.Cu") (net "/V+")))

